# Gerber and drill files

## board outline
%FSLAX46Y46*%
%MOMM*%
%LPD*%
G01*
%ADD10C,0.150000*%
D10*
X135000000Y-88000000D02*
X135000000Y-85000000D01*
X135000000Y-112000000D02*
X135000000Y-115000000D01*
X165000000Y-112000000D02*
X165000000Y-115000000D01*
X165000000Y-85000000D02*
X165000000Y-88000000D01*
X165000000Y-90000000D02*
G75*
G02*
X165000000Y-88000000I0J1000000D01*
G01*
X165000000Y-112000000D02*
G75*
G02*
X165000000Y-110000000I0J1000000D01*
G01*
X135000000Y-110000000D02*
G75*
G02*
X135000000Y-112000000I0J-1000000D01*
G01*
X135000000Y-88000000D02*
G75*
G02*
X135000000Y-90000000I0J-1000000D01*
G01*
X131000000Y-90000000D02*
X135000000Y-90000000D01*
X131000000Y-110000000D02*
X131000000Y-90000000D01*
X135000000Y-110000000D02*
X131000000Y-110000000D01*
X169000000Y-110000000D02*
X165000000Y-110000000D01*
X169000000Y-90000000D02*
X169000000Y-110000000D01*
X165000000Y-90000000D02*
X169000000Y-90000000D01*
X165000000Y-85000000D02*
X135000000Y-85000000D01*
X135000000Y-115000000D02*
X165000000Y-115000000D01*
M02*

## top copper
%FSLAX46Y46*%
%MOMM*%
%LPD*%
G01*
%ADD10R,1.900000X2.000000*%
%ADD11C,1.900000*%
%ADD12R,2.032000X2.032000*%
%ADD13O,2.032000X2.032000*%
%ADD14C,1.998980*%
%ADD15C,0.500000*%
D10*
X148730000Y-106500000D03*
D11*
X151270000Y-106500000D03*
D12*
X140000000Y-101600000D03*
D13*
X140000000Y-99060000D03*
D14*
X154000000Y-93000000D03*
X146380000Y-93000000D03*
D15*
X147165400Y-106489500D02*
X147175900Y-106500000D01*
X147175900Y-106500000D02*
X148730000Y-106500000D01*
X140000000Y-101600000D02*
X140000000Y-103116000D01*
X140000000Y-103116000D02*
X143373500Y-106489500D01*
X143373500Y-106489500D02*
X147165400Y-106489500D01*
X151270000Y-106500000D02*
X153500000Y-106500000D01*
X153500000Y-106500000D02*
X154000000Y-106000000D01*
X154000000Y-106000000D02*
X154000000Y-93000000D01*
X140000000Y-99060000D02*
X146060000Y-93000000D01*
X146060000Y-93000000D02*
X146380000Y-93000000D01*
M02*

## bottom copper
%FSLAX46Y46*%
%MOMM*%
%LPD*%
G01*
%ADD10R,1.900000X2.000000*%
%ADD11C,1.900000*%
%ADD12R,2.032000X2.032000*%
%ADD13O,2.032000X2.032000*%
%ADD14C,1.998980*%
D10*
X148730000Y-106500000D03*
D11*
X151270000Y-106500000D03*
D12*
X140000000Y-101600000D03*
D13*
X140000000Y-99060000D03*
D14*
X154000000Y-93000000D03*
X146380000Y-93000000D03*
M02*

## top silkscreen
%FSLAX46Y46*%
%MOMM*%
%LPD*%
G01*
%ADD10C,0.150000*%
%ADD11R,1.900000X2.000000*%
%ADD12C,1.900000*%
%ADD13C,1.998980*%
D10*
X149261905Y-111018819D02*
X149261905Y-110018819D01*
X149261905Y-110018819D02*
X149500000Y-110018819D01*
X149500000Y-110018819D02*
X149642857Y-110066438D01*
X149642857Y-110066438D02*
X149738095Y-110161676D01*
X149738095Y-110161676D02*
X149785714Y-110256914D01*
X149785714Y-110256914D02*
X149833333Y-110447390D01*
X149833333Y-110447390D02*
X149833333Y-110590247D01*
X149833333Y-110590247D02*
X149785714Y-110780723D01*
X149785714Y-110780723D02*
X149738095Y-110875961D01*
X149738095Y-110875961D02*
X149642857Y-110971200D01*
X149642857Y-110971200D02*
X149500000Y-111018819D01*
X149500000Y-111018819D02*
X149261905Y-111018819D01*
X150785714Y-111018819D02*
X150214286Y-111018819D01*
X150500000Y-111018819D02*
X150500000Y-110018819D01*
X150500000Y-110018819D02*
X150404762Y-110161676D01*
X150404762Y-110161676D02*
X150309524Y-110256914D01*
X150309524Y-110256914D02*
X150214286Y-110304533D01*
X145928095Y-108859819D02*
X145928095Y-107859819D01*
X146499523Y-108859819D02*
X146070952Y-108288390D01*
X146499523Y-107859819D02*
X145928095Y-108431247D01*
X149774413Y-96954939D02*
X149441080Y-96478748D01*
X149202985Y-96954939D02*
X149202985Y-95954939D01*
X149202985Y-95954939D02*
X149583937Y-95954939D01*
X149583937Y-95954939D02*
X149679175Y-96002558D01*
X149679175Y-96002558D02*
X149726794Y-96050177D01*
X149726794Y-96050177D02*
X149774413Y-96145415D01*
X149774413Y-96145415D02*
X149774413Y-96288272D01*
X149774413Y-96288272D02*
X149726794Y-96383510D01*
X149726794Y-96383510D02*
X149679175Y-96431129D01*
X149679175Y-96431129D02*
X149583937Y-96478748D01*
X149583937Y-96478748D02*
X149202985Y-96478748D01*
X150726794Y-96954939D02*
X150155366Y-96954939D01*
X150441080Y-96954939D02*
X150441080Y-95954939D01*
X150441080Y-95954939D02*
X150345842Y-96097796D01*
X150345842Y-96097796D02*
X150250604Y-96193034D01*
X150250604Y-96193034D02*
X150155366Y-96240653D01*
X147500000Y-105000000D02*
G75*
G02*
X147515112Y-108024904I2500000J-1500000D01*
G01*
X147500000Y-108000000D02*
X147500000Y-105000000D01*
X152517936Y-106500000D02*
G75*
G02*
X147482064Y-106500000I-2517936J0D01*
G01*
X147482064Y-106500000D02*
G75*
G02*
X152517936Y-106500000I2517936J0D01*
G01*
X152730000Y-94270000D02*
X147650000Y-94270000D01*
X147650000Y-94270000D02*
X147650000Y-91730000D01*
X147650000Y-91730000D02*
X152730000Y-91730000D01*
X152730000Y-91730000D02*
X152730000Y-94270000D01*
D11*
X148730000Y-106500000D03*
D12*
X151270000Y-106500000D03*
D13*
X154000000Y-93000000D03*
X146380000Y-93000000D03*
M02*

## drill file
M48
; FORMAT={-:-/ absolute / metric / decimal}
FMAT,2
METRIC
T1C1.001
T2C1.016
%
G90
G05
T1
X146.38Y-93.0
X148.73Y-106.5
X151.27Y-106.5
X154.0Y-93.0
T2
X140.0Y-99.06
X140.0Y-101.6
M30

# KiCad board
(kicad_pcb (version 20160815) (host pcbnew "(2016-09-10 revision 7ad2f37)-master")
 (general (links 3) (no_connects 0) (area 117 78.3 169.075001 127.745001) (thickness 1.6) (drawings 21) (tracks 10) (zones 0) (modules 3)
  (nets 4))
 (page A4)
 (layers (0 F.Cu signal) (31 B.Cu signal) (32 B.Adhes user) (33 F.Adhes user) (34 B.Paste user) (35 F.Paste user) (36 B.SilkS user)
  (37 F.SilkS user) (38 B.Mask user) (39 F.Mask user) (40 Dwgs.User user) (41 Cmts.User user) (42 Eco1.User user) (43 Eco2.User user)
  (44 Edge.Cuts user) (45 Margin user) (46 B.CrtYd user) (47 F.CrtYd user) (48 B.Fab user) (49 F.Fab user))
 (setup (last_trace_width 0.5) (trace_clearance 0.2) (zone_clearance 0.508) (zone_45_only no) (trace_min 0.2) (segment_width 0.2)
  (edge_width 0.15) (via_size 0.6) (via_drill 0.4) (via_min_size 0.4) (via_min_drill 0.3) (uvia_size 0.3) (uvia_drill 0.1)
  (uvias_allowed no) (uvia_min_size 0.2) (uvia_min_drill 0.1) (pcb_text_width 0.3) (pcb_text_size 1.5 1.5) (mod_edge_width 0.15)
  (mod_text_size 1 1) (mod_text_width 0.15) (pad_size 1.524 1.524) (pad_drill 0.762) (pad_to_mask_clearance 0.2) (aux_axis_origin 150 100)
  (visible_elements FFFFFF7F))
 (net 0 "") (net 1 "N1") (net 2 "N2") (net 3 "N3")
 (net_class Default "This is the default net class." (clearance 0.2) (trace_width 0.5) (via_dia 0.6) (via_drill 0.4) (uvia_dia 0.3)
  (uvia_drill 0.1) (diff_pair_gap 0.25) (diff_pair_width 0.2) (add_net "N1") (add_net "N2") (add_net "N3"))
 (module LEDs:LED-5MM (layer F.Cu) (at 150 106.5)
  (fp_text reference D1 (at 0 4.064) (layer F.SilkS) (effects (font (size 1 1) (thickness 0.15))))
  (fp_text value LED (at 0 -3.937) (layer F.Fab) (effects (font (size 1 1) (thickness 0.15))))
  (fp_arc (start 0 0) (end -2.5 -1.5) (angle 297.5) (layer F.SilkS) (width 0.15))
  (fp_line (start -2.5 1.5) (end -2.5 -1.5) (layer F.SilkS) (width 0.15))
  (fp_circle (center 0 0) (end -0.3 -2.5) (layer F.SilkS) (width 0.15))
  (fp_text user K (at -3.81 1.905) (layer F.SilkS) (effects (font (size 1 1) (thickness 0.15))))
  (pad 1 thru_hole rect (at -1.27 0 90) (size 2 1.9) (drill 1.00076) (layers *.Cu *.Mask F.SilkS) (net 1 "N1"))
  (pad 2 thru_hole circle (at 1.27 0) (size 1.9 1.9) (drill 1.00076) (layers *.Cu *.Mask F.SilkS) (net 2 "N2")))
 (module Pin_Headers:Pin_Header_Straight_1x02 (layer B.Cu) (at 140 101.6)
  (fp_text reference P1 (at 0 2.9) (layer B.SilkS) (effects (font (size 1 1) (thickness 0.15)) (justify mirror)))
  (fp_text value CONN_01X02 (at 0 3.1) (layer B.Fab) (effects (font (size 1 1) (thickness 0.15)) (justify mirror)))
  (pad 1 thru_hole rect (at 0 0) (size 2.032 2.032) (drill 1.016) (layers *.Cu *.Mask B.SilkS) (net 1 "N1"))
  (pad 2 thru_hole oval (at 0 -2.54) (size 2.032 2.032) (drill 1.016) (layers *.Cu *.Mask B.SilkS) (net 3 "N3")))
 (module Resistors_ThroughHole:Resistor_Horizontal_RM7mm (layer F.Cu) (at 154 93 180)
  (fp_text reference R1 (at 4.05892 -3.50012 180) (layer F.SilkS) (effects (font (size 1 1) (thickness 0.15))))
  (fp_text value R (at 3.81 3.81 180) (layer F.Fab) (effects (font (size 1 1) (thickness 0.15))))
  (fp_line (start 1.27 -1.27) (end 6.35 -1.27) (layer F.SilkS) (width 0.15))
  (fp_line (start 6.35 -1.27) (end 6.35 1.27) (layer F.SilkS) (width 0.15))
  (fp_line (start 6.35 1.27) (end 1.27 1.27) (layer F.SilkS) (width 0.15))
  (fp_line (start 1.27 1.27) (end 1.27 -1.27) (layer F.SilkS) (width 0.15))
  (pad 1 thru_hole circle (at 0 0 180) (size 1.99898 1.99898) (drill 1.00076) (layers *.Cu *.SilkS *.Mask) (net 2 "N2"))
  (pad 2 thru_hole circle (at 7.62 0 180) (size 1.99898 1.99898) (drill 1.00076) (layers *.Cu *.SilkS *.Mask) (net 3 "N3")))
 (gr_line (start 135 88) (end 135 85) (layer Edge.Cuts) (width 0.15))
 (gr_line (start 135 112) (end 135 115) (layer Edge.Cuts) (width 0.15))
 (gr_line (start 165 112) (end 165 115) (layer Edge.Cuts) (width 0.15))
 (gr_line (start 165 85) (end 165 88) (layer Edge.Cuts) (width 0.15))
 (gr_arc (start 165 89) (end 165 90) (angle 180) (layer Edge.Cuts) (width 0.15))
 (gr_arc (start 165 111) (end 165 112) (angle 180) (layer Edge.Cuts) (width 0.15))
 (gr_arc (start 135 111) (end 135 110) (angle 180) (layer Edge.Cuts) (width 0.15))
 (gr_arc (start 135 89) (end 135 88) (angle 180) (layer Edge.Cuts) (width 0.15))
 (gr_line (start 131 90) (end 135 90) (layer Edge.Cuts) (width 0.15))
 (gr_line (start 131 110) (end 131 90) (layer Edge.Cuts) (width 0.15))
 (gr_line (start 135 110) (end 131 110) (layer Edge.Cuts) (width 0.15))
 (gr_line (start 169 110) (end 165 110) (layer Edge.Cuts) (width 0.15))
 (gr_line (start 169 90) (end 169 110) (layer Edge.Cuts) (width 0.15))
 (gr_line (start 165 90) (end 169 90) (layer Edge.Cuts) (width 0.15))
 (gr_line (start 165 85) (end 135 85) (layer Edge.Cuts) (width 0.15))
 (gr_line (start 135 115) (end 165 115) (layer Edge.Cuts) (width 0.15))
 (segment (start 147.1654 106.4895) (end 147.1759 106.5) (width 0.5) (layer F.Cu) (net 1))
 (segment (start 147.1759 106.5) (end 148.73 106.5) (width 0.5) (layer F.Cu) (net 1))
 (segment (start 140 101.6) (end 140 103.116) (width 0.5) (layer F.Cu) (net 1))
 (segment (start 140 103.116) (end 143.3735 106.4895) (width 0.5) (layer F.Cu) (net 1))
 (segment (start 143.3735 106.4895) (end 147.1654 106.4895) (width 0.5) (layer F.Cu) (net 1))
 (segment (start 151.27 106.5) (end 153.5 106.5) (width 0.5) (layer F.Cu) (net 2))
 (segment (start 153.5 106.5) (end 154 106) (width 0.5) (layer F.Cu) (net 2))
 (segment (start 154 106) (end 154 93) (width 0.5) (layer F.Cu) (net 2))
 (segment (start 140 99.06) (end 146.06 93) (width 0.5) (layer F.Cu) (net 3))
 (segment (start 146.06 93) (end 146.38 93) (width 0.5) (layer F.Cu) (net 3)))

